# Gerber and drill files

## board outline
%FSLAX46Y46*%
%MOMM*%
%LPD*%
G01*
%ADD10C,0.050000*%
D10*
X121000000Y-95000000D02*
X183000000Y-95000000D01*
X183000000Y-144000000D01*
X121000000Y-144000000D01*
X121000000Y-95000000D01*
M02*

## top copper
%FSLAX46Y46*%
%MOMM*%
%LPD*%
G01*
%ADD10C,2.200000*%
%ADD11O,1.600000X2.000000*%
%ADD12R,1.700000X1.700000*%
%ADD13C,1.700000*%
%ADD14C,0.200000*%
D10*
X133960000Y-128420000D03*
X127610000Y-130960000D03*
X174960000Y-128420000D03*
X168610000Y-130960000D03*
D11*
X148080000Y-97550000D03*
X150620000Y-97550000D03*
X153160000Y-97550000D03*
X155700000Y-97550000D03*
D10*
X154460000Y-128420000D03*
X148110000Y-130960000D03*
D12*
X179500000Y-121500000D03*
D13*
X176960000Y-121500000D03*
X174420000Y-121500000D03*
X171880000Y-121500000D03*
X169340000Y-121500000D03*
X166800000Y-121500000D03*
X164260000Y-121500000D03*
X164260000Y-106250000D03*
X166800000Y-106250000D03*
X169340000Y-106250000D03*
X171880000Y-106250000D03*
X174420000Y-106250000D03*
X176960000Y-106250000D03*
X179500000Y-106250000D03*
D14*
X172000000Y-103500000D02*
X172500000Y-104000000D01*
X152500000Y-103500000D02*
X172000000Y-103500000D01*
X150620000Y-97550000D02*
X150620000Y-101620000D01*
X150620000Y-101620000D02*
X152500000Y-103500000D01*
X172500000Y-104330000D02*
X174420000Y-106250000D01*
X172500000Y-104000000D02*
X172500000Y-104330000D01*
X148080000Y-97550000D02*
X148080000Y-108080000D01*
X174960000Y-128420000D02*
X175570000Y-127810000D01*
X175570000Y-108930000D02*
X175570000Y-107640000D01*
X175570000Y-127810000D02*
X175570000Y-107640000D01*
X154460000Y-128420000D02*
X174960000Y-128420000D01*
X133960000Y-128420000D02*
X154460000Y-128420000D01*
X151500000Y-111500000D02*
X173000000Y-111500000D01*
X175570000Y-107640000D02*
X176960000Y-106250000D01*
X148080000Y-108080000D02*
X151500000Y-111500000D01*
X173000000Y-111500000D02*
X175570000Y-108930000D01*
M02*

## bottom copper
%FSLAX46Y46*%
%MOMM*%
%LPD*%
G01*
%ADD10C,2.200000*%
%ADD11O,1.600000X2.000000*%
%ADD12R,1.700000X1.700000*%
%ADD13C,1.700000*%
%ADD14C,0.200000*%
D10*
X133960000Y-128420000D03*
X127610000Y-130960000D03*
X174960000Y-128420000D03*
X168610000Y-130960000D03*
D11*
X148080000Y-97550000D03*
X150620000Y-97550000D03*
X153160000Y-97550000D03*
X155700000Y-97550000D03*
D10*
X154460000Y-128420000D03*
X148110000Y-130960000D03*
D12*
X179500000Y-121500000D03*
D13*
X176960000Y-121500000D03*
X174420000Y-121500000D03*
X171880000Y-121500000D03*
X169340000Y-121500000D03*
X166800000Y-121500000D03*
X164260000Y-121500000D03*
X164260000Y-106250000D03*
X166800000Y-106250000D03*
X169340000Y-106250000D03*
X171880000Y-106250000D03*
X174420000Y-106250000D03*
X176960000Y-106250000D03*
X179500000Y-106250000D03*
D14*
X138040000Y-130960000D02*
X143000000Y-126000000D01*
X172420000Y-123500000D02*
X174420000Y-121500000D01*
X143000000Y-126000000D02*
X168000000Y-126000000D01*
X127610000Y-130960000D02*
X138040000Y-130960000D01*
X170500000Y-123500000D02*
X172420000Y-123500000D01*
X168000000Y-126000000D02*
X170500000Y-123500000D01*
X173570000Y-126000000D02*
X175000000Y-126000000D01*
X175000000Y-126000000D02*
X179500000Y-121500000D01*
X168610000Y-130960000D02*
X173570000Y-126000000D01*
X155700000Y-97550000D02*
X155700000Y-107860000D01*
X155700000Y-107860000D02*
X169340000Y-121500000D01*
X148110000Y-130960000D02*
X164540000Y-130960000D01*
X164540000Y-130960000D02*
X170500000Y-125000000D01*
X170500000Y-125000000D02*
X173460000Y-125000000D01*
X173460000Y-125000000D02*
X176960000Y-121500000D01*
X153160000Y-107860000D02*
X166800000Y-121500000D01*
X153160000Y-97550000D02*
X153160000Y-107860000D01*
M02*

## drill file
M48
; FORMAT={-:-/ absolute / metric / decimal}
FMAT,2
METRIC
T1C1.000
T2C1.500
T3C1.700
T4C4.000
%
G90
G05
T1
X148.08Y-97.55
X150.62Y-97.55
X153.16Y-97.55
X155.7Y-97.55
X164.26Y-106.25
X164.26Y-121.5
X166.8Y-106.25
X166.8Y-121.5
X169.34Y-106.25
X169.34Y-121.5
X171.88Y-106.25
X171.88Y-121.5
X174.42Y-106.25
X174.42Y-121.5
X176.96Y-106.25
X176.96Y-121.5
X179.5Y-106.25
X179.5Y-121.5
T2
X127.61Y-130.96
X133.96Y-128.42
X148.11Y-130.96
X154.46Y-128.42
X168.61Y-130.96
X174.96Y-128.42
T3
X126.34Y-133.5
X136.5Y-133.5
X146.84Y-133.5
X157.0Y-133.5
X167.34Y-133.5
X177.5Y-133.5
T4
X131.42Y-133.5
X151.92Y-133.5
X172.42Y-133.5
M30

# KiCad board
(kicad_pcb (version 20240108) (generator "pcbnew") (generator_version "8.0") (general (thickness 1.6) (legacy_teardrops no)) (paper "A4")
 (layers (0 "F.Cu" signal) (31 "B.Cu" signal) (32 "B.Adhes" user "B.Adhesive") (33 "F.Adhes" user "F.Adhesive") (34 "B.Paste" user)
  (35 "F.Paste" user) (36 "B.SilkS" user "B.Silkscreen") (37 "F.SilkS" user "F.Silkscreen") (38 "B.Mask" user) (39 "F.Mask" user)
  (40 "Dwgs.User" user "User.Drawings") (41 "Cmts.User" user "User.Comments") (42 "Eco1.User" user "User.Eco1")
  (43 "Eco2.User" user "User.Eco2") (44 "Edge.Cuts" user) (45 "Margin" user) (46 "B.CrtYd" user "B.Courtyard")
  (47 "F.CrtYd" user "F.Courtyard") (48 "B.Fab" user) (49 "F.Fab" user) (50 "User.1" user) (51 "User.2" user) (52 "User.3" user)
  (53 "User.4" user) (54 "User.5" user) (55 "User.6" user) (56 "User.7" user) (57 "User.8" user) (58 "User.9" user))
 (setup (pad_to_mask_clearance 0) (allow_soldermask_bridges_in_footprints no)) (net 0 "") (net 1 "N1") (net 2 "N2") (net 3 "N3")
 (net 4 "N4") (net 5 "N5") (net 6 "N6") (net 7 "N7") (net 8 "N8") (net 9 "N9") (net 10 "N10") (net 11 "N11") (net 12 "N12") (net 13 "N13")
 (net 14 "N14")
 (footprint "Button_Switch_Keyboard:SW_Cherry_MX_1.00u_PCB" (layer "F.Cu") (at 133.96 128.42)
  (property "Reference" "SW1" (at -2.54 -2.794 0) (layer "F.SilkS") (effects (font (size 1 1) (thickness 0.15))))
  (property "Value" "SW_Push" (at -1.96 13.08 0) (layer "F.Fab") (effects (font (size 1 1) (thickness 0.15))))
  (pad "" np_thru_hole circle (at -7.62 5.08) (size 1.7 1.7) (drill 1.7) (layers "*.Cu" "*.Mask"))
  (pad "" np_thru_hole circle (at -2.54 5.08) (size 4 4) (drill 4) (layers "*.Cu" "*.Mask"))
  (pad "" np_thru_hole circle (at 2.54 5.08) (size 1.7 1.7) (drill 1.7) (layers "*.Cu" "*.Mask"))
  (pad "1" thru_hole circle (at 0 0) (size 2.2 2.2) (drill 1.5) (layers "*.Cu" "*.Mask") (remove_unused_layers no) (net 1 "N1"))
  (pad "2" thru_hole circle (at -6.35 2.54) (size 2.2 2.2) (drill 1.5) (layers "*.Cu" "*.Mask") (remove_unused_layers no) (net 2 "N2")))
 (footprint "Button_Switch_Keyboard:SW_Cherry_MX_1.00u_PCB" (layer "F.Cu") (at 174.96 128.42)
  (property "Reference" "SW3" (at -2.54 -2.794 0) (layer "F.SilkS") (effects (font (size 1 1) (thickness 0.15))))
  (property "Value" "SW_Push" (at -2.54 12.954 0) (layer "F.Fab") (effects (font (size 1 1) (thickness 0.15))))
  (pad "" np_thru_hole circle (at -7.62 5.08) (size 1.7 1.7) (drill 1.7) (layers "*.Cu" "*.Mask"))
  (pad "" np_thru_hole circle (at -2.54 5.08) (size 4 4) (drill 4) (layers "*.Cu" "*.Mask"))
  (pad "" np_thru_hole circle (at 2.54 5.08) (size 1.7 1.7) (drill 1.7) (layers "*.Cu" "*.Mask"))
  (pad "1" thru_hole circle (at 0 0) (size 2.2 2.2) (drill 1.5) (layers "*.Cu" "*.Mask") (remove_unused_layers no) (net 1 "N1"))
  (pad "2" thru_hole circle (at -6.35 2.54) (size 2.2 2.2) (drill 1.5) (layers "*.Cu" "*.Mask") (remove_unused_layers no) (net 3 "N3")))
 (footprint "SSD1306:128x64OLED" (layer "F.Cu") (at 151.7 108.15)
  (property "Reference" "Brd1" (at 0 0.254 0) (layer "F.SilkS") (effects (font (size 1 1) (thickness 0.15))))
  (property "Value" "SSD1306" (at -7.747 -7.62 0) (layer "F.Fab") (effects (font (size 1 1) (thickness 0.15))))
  (pad "1" thru_hole oval (at -3.62 -10.6 90) (size 2 1.6) (drill 1) (layers "*.Cu" "*.Mask") (remove_unused_layers no) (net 1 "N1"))
  (pad "2" thru_hole oval (at -1.08 -10.6 90) (size 2 1.6) (drill 1) (layers "*.Cu" "*.Mask") (remove_unused_layers no) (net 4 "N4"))
  (pad "3" thru_hole oval (at 1.46 -10.6 90) (size 2 1.6) (drill 1) (layers "*.Cu" "*.Mask") (remove_unused_layers no) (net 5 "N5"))
  (pad "4" thru_hole oval (at 4 -10.6 90) (size 2 1.6) (drill 1) (layers "*.Cu" "*.Mask") (remove_unused_layers no) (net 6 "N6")))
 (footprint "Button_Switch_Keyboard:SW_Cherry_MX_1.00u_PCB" (layer "F.Cu") (at 154.46 128.42)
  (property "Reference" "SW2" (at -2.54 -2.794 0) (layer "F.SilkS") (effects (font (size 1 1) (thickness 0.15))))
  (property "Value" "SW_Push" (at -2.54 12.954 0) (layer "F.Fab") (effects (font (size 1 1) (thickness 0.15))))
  (pad "" np_thru_hole circle (at -7.62 5.08) (size 1.7 1.7) (drill 1.7) (layers "*.Cu" "*.Mask"))
  (pad "" np_thru_hole circle (at -2.54 5.08) (size 4 4) (drill 4) (layers "*.Cu" "*.Mask"))
  (pad "" np_thru_hole circle (at 2.54 5.08) (size 1.7 1.7) (drill 1.7) (layers "*.Cu" "*.Mask"))
  (pad "1" thru_hole circle (at 0 0) (size 2.2 2.2) (drill 1.5) (layers "*.Cu" "*.Mask") (remove_unused_layers no) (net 1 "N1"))
  (pad "2" thru_hole circle (at -6.35 2.54) (size 2.2 2.2) (drill 1.5) (layers "*.Cu" "*.Mask") (remove_unused_layers no) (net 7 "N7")))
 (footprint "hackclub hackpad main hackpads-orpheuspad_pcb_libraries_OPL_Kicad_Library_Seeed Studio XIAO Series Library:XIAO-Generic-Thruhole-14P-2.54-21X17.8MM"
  (layer "B.Cu") (at 171.88 113.875 90)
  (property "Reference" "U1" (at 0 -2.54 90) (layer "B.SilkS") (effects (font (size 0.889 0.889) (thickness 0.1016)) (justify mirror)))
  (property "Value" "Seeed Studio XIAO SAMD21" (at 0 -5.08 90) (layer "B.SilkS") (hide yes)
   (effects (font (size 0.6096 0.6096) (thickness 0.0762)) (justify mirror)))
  (pad "1" thru_hole rect (at -7.625 7.62 90) (size 1.7 1.7) (drill 1) (layers "*.Cu" "*.Mask") (remove_unused_layers no) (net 3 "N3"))
  (pad "2" thru_hole circle (at -7.625 5.08 90) (size 1.7 1.7) (drill 1) (layers "*.Cu" "*.Mask") (remove_unused_layers no) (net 7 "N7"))
  (pad "3" thru_hole circle (at -7.625 2.54 90) (size 1.7 1.7) (drill 1) (layers "*.Cu" "*.Mask") (remove_unused_layers no) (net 2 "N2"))
  (pad "4" thru_hole circle (at -7.625 0 90) (size 1.7 1.7) (drill 1) (layers "*.Cu" "*.Mask") (remove_unused_layers no) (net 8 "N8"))
  (pad "5" thru_hole circle (at -7.625 -2.54 90) (size 1.7 1.7) (drill 1) (layers "*.Cu" "*.Mask") (remove_unused_layers no) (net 6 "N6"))
  (pad "6" thru_hole circle (at -7.625 -5.08 270) (size 1.7 1.7) (drill 1) (layers "*.Cu" "*.Mask") (remove_unused_layers no) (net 5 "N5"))
  (pad "7" thru_hole circle (at -7.625 -7.62 90) (size 1.7 1.7) (drill 1) (layers "*.Cu" "*.Mask") (remove_unused_layers no) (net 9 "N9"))
  (pad "8" thru_hole circle (at 7.625 -7.62 90) (size 1.7 1.7) (drill 1) (layers "*.Cu" "*.Mask") (remove_unused_layers no) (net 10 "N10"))
  (pad "9" thru_hole circle (at 7.625 -5.08 90) (size 1.7 1.7) (drill 1) (layers "*.Cu" "*.Mask") (remove_unused_layers no) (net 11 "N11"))
  (pad "10" thru_hole circle (at 7.625 -2.54 90) (size 1.7 1.7) (drill 1) (layers "*.Cu" "*.Mask") (remove_unused_layers no) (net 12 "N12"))
  (pad "11" thru_hole circle (at 7.625 0 90) (size 1.7 1.7) (drill 1) (layers "*.Cu" "*.Mask") (remove_unused_layers no) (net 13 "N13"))
  (pad "12" thru_hole circle (at 7.625 2.54 90) (size 1.7 1.7) (drill 1) (layers "*.Cu" "*.Mask") (remove_unused_layers no) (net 4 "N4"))
  (pad "13" thru_hole circle (at 7.625 5.08 90) (size 1.7 1.7) (drill 1) (layers "*.Cu" "*.Mask") (remove_unused_layers no) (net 1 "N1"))
  (pad "14" thru_hole circle (at 7.625 7.62 90) (size 1.7 1.7) (drill 1) (layers "*.Cu" "*.Mask") (remove_unused_layers no) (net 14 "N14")))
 (gr_rect (start 121 95) (end 183 144) (stroke (width 0.05) (type default)) (fill none) (layer "Edge.Cuts"))
 (segment (start 138.04 130.96) (end 143 126) (width 0.2) (layer "B.Cu") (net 2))
 (segment (start 172.42 123.5) (end 174.42 121.5) (width 0.2) (layer "B.Cu") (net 2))
 (segment (start 143 126) (end 168 126) (width 0.2) (layer "B.Cu") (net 2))
 (segment (start 127.61 130.96) (end 138.04 130.96) (width 0.2) (layer "B.Cu") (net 2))
 (segment (start 170.5 123.5) (end 172.42 123.5) (width 0.2) (layer "B.Cu") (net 2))
 (segment (start 168 126) (end 170.5 123.5) (width 0.2) (layer "B.Cu") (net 2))
 (segment (start 172 103.5) (end 172.5 104) (width 0.2) (layer "F.Cu") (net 4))
 (segment (start 152.5 103.5) (end 172 103.5) (width 0.2) (layer "F.Cu") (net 4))
 (segment (start 150.62 97.55) (end 150.62 101.62) (width 0.2) (layer "F.Cu") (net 4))
 (segment (start 150.62 101.62) (end 152.5 103.5) (width 0.2) (layer "F.Cu") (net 4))
 (segment (start 172.5 104.33) (end 174.42 106.25) (width 0.2) (layer "F.Cu") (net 4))
 (segment (start 172.5 104) (end 172.5 104.33) (width 0.2) (layer "F.Cu") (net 4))
 (segment (start 173.57 126) (end 175 126) (width 0.2) (layer "B.Cu") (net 3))
 (segment (start 175 126) (end 179.5 121.5) (width 0.2) (layer "B.Cu") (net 3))
 (segment (start 168.61 130.96) (end 173.57 126) (width 0.2) (layer "B.Cu") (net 3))
 (segment (start 148.08 97.55) (end 148.08 108.08) (width 0.2) (layer "F.Cu") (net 1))
 (segment (start 174.96 128.42) (end 175.57 127.81) (width 0.2) (layer "F.Cu") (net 1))
 (segment (start 175.57 108.93) (end 175.57 107.64) (width 0.2) (layer "F.Cu") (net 1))
 (segment (start 175.57 127.81) (end 175.57 107.64) (width 0.2) (layer "F.Cu") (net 1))
 (segment (start 154.46 128.42) (end 174.96 128.42) (width 0.2) (layer "F.Cu") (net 1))
 (segment (start 133.96 128.42) (end 154.46 128.42) (width 0.2) (layer "F.Cu") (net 1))
 (segment (start 151.5 111.5) (end 173 111.5) (width 0.2) (layer "F.Cu") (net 1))
 (segment (start 175.57 107.64) (end 176.96 106.25) (width 0.2) (layer "F.Cu") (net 1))
 (segment (start 148.08 108.08) (end 151.5 111.5) (width 0.2) (layer "F.Cu") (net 1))
 (segment (start 173 111.5) (end 175.57 108.93) (width 0.2) (layer "F.Cu") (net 1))
 (segment (start 155.7 97.55) (end 155.7 107.86) (width 0.2) (layer "B.Cu") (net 6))
 (segment (start 155.7 107.86) (end 169.34 121.5) (width 0.2) (layer "B.Cu") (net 6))
 (segment (start 148.11 130.96) (end 164.54 130.96) (width 0.2) (layer "B.Cu") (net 7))
 (segment (start 164.54 130.96) (end 170.5 125) (width 0.2) (layer "B.Cu") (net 7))
 (segment (start 170.5 125) (end 173.46 125) (width 0.2) (layer "B.Cu") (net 7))
 (segment (start 173.46 125) (end 176.96 121.5) (width 0.2) (layer "B.Cu") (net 7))
 (segment (start 153.16 107.86) (end 166.8 121.5) (width 0.2) (layer "B.Cu") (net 5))
 (segment (start 153.16 97.55) (end 153.16 107.86) (width 0.2) (layer "B.Cu") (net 5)))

